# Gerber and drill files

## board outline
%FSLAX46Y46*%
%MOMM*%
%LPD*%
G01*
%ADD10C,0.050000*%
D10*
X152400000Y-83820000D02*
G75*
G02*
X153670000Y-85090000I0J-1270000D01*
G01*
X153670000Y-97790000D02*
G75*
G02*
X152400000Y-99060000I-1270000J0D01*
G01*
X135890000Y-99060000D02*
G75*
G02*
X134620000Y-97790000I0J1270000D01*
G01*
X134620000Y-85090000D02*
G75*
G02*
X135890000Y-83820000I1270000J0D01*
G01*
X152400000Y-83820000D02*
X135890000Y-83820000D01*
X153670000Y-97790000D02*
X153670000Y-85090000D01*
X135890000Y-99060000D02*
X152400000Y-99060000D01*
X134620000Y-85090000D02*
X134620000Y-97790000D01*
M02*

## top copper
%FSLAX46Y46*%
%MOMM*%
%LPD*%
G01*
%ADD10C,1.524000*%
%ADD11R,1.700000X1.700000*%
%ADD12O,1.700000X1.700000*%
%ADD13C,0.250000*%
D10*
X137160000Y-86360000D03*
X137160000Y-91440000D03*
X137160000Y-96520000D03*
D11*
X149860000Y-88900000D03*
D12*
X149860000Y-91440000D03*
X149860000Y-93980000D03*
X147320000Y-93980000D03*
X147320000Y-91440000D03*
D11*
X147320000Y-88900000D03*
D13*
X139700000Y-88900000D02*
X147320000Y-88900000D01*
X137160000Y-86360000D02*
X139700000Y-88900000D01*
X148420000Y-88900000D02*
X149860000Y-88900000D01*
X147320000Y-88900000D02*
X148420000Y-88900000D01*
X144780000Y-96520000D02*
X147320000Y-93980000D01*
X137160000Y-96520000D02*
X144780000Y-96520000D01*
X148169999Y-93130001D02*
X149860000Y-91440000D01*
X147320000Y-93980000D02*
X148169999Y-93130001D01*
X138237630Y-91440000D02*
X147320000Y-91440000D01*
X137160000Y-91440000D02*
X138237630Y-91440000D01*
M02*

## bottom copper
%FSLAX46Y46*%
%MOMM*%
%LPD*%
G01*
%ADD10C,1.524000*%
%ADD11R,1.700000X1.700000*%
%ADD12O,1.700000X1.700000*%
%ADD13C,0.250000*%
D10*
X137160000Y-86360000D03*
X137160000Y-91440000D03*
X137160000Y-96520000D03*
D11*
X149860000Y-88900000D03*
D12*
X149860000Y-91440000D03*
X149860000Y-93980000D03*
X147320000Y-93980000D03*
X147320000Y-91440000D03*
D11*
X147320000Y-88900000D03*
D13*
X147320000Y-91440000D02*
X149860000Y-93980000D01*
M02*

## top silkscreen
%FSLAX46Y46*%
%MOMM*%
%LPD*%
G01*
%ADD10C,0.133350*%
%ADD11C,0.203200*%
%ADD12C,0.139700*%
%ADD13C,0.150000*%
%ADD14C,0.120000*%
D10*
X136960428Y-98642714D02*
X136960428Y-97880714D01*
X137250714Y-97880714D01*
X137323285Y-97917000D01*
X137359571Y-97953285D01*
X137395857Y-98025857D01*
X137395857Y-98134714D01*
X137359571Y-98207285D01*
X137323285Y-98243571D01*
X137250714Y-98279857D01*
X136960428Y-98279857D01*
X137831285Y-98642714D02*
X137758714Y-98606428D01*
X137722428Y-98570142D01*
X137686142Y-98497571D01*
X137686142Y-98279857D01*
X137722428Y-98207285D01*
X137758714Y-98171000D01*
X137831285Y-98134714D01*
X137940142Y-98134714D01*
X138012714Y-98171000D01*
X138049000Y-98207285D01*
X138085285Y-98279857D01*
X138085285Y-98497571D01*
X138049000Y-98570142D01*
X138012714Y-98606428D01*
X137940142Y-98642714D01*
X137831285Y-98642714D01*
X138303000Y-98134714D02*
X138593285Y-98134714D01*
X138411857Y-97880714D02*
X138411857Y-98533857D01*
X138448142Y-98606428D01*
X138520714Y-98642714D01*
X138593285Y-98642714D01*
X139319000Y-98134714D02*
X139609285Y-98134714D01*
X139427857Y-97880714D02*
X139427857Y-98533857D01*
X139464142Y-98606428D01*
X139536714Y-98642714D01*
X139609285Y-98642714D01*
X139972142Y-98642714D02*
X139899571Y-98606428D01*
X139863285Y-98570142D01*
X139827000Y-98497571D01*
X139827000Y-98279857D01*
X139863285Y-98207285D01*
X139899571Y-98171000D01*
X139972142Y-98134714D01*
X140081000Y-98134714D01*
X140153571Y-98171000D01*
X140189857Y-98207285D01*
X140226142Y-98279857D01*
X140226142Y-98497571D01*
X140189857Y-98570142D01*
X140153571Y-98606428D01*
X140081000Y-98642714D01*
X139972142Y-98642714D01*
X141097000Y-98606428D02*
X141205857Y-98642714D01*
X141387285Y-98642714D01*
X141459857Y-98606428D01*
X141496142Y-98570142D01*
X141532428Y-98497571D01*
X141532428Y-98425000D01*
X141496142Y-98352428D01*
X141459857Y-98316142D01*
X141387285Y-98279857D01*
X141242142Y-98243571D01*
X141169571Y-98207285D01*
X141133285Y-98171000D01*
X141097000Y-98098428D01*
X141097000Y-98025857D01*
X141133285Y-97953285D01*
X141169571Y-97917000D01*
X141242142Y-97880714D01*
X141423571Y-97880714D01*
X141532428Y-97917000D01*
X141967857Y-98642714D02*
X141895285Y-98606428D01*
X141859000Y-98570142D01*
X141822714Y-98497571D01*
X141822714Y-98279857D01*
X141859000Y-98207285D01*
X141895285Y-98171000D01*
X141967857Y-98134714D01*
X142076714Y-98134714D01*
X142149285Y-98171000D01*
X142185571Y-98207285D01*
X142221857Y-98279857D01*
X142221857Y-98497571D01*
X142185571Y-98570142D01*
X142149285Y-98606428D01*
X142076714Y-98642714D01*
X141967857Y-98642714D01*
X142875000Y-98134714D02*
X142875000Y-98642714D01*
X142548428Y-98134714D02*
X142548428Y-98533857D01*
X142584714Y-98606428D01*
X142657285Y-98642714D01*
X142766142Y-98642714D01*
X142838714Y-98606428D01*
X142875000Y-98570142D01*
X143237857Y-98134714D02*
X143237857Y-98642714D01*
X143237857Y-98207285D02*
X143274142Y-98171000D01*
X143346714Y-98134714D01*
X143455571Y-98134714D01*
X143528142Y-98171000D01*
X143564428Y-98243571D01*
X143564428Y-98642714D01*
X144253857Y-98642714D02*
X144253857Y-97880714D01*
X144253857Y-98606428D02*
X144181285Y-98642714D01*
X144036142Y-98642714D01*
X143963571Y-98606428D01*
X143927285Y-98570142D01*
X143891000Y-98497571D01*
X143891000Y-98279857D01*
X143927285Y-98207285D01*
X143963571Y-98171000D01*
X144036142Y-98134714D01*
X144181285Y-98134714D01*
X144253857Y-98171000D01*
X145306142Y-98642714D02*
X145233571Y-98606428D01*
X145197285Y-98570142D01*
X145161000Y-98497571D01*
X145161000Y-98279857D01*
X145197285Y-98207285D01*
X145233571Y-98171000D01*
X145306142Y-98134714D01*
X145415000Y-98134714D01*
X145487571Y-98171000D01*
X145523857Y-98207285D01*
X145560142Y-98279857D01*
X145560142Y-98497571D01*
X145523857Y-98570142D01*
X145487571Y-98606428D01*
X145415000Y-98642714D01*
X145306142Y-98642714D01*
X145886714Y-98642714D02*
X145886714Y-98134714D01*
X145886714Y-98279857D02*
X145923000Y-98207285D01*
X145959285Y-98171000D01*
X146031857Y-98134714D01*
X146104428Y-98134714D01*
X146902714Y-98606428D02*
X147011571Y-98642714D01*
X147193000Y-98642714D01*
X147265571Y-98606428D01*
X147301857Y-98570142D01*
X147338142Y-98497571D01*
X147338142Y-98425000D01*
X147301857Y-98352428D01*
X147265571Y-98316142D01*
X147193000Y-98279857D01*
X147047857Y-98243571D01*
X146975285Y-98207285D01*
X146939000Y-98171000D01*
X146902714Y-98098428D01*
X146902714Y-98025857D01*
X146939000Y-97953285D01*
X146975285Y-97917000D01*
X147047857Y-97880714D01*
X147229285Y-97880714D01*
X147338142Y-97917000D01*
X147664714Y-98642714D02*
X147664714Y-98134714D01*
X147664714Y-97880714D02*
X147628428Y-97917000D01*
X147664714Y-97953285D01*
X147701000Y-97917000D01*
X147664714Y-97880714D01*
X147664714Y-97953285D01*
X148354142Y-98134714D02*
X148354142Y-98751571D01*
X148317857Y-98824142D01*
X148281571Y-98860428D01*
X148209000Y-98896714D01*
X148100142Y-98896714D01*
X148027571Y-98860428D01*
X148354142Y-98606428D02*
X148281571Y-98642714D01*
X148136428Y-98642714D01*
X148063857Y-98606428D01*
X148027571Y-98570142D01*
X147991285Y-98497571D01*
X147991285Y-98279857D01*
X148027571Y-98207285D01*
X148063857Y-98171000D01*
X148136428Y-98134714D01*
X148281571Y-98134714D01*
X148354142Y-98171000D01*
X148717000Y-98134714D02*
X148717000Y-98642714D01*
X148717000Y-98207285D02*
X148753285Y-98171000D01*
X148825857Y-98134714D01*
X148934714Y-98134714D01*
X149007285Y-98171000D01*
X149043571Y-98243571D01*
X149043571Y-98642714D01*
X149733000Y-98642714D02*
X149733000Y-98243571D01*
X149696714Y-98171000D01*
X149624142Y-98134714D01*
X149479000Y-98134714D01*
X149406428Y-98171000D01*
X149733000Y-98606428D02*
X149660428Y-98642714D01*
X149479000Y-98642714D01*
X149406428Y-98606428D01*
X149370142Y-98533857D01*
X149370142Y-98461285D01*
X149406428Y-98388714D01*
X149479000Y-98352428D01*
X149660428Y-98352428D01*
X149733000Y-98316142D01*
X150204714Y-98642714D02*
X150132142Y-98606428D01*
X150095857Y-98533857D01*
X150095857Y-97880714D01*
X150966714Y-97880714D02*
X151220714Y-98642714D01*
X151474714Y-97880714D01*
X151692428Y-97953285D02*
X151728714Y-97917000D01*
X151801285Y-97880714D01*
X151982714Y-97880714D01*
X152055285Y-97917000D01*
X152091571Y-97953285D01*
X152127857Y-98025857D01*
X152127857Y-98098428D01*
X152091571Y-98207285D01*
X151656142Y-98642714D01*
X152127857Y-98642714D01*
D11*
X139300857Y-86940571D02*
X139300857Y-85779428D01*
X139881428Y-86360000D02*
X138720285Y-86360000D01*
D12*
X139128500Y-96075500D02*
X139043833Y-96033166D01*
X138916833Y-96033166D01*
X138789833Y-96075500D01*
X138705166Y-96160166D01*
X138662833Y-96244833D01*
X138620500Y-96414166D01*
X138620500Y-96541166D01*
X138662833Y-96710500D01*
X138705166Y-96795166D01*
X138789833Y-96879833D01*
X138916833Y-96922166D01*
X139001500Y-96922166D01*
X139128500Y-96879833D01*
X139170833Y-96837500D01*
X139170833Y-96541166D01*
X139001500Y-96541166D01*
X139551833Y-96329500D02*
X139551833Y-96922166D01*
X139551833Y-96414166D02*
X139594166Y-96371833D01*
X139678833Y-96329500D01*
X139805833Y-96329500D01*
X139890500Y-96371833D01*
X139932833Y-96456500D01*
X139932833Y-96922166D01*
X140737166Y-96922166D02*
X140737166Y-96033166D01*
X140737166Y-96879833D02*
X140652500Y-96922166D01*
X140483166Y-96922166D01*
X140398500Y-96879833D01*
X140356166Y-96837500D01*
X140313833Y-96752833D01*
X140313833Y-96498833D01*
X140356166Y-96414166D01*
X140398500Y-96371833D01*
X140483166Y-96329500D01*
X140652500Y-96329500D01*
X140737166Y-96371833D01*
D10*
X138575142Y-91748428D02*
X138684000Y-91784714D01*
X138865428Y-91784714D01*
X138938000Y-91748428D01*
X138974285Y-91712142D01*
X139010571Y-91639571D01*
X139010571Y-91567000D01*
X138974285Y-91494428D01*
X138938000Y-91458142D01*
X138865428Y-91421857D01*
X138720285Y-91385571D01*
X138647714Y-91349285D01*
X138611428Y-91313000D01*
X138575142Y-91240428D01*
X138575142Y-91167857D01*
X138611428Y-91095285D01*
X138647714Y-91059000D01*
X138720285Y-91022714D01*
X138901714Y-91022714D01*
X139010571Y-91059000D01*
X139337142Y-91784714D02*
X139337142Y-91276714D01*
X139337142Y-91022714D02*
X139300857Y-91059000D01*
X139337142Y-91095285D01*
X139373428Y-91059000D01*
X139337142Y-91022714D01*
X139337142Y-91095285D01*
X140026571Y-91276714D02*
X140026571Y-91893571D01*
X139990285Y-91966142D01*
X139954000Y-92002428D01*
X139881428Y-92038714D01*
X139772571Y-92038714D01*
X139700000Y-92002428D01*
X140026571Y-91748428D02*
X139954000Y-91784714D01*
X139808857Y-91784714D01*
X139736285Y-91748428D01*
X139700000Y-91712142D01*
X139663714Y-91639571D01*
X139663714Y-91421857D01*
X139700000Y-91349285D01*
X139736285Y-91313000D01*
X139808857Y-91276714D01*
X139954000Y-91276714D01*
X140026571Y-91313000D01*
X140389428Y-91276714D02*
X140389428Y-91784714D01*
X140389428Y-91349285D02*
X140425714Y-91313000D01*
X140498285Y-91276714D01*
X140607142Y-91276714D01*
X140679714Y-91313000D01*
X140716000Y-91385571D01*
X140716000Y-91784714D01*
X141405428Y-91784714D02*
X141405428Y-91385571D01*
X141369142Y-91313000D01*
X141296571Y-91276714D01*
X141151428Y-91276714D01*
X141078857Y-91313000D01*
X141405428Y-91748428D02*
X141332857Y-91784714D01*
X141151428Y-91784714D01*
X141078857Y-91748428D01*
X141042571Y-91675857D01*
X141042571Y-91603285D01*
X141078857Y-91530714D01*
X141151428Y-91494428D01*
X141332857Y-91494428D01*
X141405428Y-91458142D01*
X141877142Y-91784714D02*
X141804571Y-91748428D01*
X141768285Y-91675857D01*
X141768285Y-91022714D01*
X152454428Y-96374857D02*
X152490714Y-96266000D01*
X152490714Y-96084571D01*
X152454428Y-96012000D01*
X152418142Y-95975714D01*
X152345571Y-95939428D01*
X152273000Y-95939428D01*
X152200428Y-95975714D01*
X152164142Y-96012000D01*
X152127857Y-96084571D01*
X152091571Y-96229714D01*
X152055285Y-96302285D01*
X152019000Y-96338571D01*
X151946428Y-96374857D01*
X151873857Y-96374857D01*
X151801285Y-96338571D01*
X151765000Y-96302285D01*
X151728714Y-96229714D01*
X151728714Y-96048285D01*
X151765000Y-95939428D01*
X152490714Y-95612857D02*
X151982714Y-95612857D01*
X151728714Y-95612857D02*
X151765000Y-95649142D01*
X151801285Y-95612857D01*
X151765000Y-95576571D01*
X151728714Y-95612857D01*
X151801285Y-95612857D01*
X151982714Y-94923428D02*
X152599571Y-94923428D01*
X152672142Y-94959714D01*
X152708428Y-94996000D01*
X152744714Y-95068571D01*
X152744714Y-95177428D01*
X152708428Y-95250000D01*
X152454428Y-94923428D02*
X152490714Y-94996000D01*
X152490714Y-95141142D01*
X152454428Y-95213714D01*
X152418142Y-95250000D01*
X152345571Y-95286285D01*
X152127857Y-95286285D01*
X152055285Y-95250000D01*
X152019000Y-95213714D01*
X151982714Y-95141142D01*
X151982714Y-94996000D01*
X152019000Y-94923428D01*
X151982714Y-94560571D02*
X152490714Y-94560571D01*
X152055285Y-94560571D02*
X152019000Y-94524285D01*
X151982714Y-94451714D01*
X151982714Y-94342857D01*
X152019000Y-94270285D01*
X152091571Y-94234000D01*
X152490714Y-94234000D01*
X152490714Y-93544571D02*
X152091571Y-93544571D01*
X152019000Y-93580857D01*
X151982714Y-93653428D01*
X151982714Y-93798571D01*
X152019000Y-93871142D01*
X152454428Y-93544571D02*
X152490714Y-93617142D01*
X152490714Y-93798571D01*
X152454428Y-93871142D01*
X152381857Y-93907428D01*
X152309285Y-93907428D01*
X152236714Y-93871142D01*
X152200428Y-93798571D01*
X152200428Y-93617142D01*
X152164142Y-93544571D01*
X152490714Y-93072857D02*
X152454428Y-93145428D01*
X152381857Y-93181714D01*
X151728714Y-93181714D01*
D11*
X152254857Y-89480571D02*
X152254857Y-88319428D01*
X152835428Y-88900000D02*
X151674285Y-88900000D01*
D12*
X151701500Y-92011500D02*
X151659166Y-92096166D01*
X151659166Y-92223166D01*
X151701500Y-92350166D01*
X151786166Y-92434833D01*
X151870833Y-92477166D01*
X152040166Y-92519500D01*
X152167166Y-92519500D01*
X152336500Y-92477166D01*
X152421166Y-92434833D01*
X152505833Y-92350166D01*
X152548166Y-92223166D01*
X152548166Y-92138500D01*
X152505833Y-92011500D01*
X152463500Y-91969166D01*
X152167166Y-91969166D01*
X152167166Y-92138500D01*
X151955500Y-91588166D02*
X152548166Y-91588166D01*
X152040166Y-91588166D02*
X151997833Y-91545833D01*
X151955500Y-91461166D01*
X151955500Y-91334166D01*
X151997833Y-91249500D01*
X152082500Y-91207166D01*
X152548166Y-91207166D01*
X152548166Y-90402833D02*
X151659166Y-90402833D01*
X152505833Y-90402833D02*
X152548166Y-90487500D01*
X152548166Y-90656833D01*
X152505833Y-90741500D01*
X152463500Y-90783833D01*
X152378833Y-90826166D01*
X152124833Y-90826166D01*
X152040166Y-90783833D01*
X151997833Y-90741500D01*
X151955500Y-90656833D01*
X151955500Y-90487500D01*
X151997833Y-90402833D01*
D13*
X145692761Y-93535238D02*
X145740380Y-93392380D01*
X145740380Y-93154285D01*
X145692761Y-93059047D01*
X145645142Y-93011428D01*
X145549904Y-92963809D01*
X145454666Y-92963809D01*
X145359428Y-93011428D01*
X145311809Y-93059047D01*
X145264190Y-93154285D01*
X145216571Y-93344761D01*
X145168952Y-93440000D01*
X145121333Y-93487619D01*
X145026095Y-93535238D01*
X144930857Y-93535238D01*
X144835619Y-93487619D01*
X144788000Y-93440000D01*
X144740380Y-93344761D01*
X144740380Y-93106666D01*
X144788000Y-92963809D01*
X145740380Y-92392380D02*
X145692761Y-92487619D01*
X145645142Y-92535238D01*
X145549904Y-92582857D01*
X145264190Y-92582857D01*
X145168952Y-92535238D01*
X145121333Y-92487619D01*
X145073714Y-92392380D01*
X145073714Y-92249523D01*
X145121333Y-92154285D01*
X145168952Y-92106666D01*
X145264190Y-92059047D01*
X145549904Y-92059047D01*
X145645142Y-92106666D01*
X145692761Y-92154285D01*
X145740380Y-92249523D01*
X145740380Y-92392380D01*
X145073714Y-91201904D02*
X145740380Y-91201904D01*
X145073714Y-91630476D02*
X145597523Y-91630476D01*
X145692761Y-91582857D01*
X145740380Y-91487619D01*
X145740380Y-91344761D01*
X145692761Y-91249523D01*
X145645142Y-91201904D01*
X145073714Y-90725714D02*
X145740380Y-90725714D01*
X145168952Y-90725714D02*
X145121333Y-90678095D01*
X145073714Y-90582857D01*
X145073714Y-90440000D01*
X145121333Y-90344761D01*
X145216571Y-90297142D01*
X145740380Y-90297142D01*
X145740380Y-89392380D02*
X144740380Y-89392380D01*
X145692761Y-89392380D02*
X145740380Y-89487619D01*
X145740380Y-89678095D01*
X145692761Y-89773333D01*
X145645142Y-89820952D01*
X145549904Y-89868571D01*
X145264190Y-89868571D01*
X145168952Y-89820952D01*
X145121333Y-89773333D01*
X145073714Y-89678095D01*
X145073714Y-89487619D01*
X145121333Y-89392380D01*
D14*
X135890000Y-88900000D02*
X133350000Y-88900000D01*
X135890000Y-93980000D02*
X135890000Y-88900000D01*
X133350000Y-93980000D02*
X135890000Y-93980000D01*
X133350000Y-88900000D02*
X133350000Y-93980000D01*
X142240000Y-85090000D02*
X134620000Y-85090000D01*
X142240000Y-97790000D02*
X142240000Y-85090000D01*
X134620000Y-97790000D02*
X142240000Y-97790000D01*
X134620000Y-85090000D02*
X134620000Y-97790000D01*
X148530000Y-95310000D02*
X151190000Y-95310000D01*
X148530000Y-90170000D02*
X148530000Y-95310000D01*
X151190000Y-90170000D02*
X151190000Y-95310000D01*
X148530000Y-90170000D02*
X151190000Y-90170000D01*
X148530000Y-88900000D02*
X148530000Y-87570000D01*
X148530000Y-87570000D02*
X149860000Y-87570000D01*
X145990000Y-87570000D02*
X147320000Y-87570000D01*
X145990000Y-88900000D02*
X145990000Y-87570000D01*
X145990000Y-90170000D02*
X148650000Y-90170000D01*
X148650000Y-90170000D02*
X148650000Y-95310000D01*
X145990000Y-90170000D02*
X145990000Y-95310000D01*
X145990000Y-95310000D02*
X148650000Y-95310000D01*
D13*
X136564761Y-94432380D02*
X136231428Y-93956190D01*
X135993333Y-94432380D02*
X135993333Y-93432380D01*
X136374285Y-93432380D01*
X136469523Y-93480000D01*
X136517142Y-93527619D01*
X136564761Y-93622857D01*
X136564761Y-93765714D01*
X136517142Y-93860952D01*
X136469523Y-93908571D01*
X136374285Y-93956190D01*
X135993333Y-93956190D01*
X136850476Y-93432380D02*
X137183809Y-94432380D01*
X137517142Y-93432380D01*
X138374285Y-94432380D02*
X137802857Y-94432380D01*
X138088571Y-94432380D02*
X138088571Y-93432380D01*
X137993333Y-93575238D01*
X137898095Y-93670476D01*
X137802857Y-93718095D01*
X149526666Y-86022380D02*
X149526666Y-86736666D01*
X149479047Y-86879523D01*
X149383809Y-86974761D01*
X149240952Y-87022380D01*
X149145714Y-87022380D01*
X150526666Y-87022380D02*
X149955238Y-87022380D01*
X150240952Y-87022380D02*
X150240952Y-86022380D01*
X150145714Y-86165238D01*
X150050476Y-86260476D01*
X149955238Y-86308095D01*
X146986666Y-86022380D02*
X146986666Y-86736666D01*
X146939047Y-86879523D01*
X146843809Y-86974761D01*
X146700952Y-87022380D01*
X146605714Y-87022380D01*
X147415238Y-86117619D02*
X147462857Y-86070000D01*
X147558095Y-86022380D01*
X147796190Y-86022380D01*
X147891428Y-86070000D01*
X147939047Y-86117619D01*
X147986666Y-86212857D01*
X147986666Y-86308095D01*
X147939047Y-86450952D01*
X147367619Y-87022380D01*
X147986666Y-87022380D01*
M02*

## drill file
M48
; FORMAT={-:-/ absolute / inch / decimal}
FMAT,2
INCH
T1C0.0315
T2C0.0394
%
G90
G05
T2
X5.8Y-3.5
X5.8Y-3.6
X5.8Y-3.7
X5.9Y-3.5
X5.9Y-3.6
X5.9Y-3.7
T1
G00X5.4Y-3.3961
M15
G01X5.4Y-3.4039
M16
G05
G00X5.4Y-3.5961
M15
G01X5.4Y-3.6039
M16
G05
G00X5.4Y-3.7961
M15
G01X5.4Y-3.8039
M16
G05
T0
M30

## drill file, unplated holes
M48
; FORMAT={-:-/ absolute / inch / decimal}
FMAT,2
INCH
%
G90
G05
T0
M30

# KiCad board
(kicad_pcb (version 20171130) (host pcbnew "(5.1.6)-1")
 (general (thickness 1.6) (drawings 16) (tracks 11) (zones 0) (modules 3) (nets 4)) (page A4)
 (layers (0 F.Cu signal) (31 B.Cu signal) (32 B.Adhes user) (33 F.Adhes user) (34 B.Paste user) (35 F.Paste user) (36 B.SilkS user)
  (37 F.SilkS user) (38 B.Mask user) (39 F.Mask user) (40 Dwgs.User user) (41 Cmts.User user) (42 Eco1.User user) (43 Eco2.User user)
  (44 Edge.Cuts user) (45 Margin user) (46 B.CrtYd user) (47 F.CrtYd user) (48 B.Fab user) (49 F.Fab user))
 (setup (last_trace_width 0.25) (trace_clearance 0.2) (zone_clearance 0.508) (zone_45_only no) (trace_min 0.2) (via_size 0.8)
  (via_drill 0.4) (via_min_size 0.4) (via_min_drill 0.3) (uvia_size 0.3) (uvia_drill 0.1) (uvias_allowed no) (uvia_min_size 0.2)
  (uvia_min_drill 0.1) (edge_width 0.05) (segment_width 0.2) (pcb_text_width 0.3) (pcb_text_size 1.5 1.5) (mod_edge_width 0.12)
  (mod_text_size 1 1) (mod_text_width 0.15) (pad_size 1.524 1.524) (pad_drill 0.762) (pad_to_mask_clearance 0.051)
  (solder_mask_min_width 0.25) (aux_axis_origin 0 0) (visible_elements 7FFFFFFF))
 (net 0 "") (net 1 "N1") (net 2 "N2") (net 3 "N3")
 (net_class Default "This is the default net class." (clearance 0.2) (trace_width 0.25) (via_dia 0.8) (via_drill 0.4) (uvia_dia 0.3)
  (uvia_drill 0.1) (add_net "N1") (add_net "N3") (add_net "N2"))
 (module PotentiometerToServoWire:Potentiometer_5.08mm (layer F.Cu) (at 137.16 91.44)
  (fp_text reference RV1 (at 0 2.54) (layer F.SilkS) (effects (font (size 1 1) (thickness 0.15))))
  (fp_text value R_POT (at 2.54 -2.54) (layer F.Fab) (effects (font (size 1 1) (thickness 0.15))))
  (fp_line (start -1.27 -2.54) (end -3.81 -2.54) (layer F.SilkS) (width 0.12))
  (fp_line (start -1.27 2.54) (end -1.27 -2.54) (layer F.SilkS) (width 0.12))
  (fp_line (start -3.81 2.54) (end -1.27 2.54) (layer F.SilkS) (width 0.12))
  (fp_line (start -3.81 -2.54) (end -3.81 2.54) (layer F.SilkS) (width 0.12))
  (fp_line (start 5.08 -6.35) (end -2.54 -6.35) (layer F.SilkS) (width 0.12))
  (fp_line (start 5.08 6.35) (end 5.08 -6.35) (layer F.SilkS) (width 0.12))
  (fp_line (start -2.54 6.35) (end 5.08 6.35) (layer F.SilkS) (width 0.12))
  (fp_line (start -2.54 -6.35) (end -2.54 6.35) (layer F.SilkS) (width 0.12))
  (pad 3 thru_hole circle (at 0 -5.08) (size 1.524 1.524) (drill oval 0.8 1) (layers *.Cu *.Mask) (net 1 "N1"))
  (pad 2 thru_hole circle (at 0 0) (size 1.524 1.524) (drill oval 0.8 1) (layers *.Cu *.Mask) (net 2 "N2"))
  (pad 1 thru_hole circle (at 0 5.08) (size 1.524 1.524) (drill oval 0.8 1) (layers *.Cu *.Mask) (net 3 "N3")))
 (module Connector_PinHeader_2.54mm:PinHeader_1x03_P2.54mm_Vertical (layer F.Cu) (at 149.86 88.9)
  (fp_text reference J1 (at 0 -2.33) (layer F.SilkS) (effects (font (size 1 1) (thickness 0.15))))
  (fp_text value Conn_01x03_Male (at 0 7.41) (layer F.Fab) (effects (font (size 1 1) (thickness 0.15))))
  (fp_line (start -1.33 6.41) (end 1.33 6.41) (layer F.SilkS) (width 0.12))
  (fp_line (start -1.33 1.27) (end -1.33 6.41) (layer F.SilkS) (width 0.12))
  (fp_line (start 1.33 1.27) (end 1.33 6.41) (layer F.SilkS) (width 0.12))
  (fp_line (start -1.33 1.27) (end 1.33 1.27) (layer F.SilkS) (width 0.12))
  (fp_line (start -1.33 0) (end -1.33 -1.33) (layer F.SilkS) (width 0.12))
  (fp_line (start -1.33 -1.33) (end 0 -1.33) (layer F.SilkS) (width 0.12))
  (pad 1 thru_hole rect (at 0 0) (size 1.7 1.7) (drill 1) (layers *.Cu *.Mask) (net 1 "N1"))
  (pad 2 thru_hole oval (at 0 2.54) (size 1.7 1.7) (drill 1) (layers *.Cu *.Mask) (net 3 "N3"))
  (pad 3 thru_hole oval (at 0 5.08) (size 1.7 1.7) (drill 1) (layers *.Cu *.Mask) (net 2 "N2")))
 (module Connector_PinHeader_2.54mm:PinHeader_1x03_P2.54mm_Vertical (layer F.Cu) (at 147.32 88.9)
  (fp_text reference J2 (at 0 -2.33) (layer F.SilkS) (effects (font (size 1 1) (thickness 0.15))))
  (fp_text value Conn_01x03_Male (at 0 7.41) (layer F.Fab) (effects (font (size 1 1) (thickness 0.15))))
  (fp_line (start -1.33 -1.33) (end 0 -1.33) (layer F.SilkS) (width 0.12))
  (fp_line (start -1.33 0) (end -1.33 -1.33) (layer F.SilkS) (width 0.12))
  (fp_line (start -1.33 1.27) (end 1.33 1.27) (layer F.SilkS) (width 0.12))
  (fp_line (start 1.33 1.27) (end 1.33 6.41) (layer F.SilkS) (width 0.12))
  (fp_line (start -1.33 1.27) (end -1.33 6.41) (layer F.SilkS) (width 0.12))
  (fp_line (start -1.33 6.41) (end 1.33 6.41) (layer F.SilkS) (width 0.12))
  (pad 3 thru_hole oval (at 0 5.08) (size 1.7 1.7) (drill 1) (layers *.Cu *.Mask) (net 3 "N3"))
  (pad 2 thru_hole oval (at 0 2.54) (size 1.7 1.7) (drill 1) (layers *.Cu *.Mask) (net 2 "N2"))
  (pad 1 thru_hole rect (at 0 0) (size 1.7 1.7) (drill 1) (layers *.Cu *.Mask) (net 1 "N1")))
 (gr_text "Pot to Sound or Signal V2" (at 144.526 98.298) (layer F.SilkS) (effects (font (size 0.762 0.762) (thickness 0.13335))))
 (gr_arc (start 152.4 85.09) (end 153.67 85.09) (angle -90) (layer Edge.Cuts) (width 0.05))
 (gr_arc (start 152.4 97.79) (end 152.4 99.06) (angle -90) (layer Edge.Cuts) (width 0.05))
 (gr_arc (start 135.89 97.79) (end 134.62 97.79) (angle -90) (layer Edge.Cuts) (width 0.05))
 (gr_arc (start 135.89 85.09) (end 135.89 83.82) (angle -90) (layer Edge.Cuts) (width 0.05))
 (gr_line (start 152.4 83.82) (end 135.89 83.82) (layer Edge.Cuts) (width 0.05))
 (gr_line (start 153.67 97.79) (end 153.67 85.09) (layer Edge.Cuts) (width 0.05))
 (gr_line (start 135.89 99.06) (end 152.4 99.06) (layer Edge.Cuts) (width 0.05))
 (gr_line (start 134.62 85.09) (end 134.62 97.79) (layer Edge.Cuts) (width 0.05))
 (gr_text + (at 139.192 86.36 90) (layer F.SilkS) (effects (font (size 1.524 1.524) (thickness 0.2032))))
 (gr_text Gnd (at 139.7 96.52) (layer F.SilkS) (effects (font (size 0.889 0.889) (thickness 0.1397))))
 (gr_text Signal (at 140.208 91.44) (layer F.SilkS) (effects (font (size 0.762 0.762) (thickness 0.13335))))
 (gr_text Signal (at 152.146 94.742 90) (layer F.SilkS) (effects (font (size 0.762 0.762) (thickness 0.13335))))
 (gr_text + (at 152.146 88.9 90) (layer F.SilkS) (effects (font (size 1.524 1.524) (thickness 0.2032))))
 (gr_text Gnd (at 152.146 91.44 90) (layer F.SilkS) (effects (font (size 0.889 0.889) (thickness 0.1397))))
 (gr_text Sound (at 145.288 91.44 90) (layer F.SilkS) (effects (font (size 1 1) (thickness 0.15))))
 (segment (start 139.7 88.9) (end 147.32 88.9) (width 0.25) (layer F.Cu) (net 1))
 (segment (start 137.16 86.36) (end 139.7 88.9) (width 0.25) (layer F.Cu) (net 1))
 (segment (start 148.42 88.9) (end 149.86 88.9) (width 0.25) (layer F.Cu) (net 1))
 (segment (start 147.32 88.9) (end 148.42 88.9) (width 0.25) (layer F.Cu) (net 1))
 (segment (start 144.78 96.52) (end 147.32 93.98) (width 0.25) (layer F.Cu) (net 3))
 (segment (start 137.16 96.52) (end 144.78 96.52) (width 0.25) (layer F.Cu) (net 3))
 (segment (start 148.169999 93.130001) (end 149.86 91.44) (width 0.25) (layer F.Cu) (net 3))
 (segment (start 147.32 93.98) (end 148.169999 93.130001) (width 0.25) (layer F.Cu) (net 3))
 (segment (start 138.23763 91.44) (end 147.32 91.44) (width 0.25) (layer F.Cu) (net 2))
 (segment (start 137.16 91.44) (end 138.23763 91.44) (width 0.25) (layer F.Cu) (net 2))
 (segment (start 147.32 91.44) (end 149.86 93.98) (width 0.25) (layer B.Cu) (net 2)))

